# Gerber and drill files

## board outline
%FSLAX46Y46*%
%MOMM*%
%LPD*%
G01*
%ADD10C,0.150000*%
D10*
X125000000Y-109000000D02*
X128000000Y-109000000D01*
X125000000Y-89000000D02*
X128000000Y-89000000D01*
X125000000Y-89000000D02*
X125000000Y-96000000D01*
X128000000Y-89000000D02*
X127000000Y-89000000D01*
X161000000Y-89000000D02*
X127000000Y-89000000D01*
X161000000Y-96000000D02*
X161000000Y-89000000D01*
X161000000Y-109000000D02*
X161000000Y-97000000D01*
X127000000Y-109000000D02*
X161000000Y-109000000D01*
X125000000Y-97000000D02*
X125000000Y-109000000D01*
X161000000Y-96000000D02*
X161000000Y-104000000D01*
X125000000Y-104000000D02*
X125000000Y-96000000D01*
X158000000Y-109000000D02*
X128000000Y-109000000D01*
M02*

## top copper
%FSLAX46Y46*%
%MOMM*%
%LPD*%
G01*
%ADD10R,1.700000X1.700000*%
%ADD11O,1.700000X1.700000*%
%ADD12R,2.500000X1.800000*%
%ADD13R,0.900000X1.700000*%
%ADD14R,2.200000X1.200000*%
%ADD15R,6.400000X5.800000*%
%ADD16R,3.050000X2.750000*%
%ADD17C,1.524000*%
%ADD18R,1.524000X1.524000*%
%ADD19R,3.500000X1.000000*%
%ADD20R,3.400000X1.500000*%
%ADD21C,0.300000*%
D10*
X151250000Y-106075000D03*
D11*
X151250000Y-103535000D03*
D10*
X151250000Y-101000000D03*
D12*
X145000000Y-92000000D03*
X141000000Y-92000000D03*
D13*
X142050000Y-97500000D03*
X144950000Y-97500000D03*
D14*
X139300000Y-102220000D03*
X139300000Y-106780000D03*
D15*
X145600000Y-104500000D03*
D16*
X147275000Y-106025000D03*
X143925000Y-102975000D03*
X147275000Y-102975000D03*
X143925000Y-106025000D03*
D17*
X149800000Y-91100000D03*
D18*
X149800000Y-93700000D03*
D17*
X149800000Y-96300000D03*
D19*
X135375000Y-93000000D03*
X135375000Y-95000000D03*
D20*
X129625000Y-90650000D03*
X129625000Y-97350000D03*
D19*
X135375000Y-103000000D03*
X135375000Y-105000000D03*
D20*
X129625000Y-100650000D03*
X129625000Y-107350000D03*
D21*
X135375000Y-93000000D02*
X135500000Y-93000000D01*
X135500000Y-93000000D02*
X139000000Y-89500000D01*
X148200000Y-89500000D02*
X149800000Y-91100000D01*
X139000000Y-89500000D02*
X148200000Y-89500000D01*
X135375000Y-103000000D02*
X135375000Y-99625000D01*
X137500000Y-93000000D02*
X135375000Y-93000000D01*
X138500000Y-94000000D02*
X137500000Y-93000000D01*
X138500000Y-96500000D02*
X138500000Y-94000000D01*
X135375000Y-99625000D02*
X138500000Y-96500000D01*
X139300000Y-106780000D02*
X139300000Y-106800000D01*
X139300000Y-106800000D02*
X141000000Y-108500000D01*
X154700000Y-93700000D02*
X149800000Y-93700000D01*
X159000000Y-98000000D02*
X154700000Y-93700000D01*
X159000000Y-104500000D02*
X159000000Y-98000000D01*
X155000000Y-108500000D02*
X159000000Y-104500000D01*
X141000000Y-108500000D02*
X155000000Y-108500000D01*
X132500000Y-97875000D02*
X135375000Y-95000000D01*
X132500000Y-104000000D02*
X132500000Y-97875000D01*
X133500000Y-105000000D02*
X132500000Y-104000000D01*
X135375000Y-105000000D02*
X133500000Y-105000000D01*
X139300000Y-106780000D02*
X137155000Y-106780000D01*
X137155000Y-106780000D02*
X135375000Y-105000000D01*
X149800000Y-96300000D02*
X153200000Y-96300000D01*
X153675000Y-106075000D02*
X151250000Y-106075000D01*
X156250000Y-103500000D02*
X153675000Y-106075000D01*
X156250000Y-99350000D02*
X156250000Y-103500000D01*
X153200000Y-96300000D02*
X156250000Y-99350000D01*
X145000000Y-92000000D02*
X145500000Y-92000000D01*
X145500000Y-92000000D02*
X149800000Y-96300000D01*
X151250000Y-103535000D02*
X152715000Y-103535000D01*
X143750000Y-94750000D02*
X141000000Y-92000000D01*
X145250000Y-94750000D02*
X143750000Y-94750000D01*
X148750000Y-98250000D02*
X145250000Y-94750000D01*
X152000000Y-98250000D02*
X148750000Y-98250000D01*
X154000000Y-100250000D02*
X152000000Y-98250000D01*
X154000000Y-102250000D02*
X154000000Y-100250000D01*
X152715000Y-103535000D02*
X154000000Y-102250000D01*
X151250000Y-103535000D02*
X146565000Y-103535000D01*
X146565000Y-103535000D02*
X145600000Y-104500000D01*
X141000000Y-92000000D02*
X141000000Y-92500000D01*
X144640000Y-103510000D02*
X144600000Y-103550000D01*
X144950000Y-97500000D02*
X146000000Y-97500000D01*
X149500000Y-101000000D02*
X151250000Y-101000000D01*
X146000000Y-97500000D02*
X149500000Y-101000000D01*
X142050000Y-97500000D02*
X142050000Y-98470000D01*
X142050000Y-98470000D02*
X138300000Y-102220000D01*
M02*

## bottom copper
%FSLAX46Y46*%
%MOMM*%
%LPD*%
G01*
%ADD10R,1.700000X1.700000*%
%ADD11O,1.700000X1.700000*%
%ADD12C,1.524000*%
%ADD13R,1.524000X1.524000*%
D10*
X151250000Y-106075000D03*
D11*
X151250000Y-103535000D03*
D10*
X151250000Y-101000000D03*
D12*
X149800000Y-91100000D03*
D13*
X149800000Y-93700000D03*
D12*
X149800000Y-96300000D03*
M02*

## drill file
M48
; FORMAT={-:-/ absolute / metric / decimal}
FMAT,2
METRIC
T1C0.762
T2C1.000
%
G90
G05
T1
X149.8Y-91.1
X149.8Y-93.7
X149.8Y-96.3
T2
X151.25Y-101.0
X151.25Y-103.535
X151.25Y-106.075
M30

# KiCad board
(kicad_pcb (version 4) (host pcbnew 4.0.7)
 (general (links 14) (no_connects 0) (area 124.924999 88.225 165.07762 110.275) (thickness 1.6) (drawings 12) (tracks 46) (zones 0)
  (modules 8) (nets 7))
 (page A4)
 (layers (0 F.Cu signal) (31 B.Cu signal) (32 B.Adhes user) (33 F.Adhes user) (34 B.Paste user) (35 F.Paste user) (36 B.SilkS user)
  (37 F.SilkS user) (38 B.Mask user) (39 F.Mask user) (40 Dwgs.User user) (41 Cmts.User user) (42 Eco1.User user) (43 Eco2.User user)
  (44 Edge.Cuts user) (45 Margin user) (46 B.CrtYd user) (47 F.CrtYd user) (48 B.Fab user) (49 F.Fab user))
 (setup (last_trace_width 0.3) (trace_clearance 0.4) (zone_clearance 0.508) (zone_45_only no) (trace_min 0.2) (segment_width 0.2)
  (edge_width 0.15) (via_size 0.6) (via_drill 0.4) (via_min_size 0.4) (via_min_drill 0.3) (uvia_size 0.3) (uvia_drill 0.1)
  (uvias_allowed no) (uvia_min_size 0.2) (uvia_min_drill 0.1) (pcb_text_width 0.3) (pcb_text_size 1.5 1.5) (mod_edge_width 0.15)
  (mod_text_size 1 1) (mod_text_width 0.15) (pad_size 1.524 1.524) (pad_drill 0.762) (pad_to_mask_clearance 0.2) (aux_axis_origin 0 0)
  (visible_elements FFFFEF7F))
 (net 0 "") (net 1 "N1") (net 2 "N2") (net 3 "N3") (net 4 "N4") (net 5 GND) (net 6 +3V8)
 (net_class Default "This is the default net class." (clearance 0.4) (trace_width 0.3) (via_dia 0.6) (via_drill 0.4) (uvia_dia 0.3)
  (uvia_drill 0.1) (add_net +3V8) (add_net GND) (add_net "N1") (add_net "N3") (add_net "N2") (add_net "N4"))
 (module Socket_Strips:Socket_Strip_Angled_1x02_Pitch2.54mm (layer F.Cu) (at 151.25 106.075 180)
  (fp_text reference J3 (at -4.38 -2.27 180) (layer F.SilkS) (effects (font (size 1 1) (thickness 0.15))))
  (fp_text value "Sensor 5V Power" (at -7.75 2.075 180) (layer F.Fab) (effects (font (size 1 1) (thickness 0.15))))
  (pad 1 thru_hole rect (at 0 0 180) (size 1.7 1.7) (drill 1) (layers *.Cu *.Mask) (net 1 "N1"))
  (pad 2 thru_hole oval (at 0 2.54 180) (size 1.7 1.7) (drill 1) (layers *.Cu *.Mask)))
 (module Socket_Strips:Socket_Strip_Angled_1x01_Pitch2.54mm (layer F.Cu) (at 151.25 101 180)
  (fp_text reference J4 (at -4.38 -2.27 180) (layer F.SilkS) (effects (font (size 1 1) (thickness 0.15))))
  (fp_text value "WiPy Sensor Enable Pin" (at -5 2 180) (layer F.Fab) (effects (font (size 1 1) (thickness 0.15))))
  (pad 1 thru_hole rect (at 0 0 180) (size 1.7 1.7) (drill 1) (layers *.Cu *.Mask) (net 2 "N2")))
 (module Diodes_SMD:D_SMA (layer F.Cu) (at 143 92 180)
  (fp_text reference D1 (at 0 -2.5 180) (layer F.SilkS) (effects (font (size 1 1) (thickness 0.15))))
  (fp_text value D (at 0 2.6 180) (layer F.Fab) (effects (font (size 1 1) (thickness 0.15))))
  (pad 1 smd rect (at -2 0 180) (size 2.5 1.8) (layers F.Cu F.Paste F.Mask) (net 1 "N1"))
  (pad 2 smd rect (at 2 0 180) (size 2.5 1.8) (layers F.Cu F.Paste F.Mask) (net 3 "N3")))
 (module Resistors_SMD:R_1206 (layer F.Cu) (at 143.5 97.5)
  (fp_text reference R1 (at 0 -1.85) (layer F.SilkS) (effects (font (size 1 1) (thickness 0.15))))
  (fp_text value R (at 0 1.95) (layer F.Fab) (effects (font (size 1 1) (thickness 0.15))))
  (pad 1 smd rect (at -1.45 0) (size 0.9 1.7) (layers F.Cu F.Paste F.Mask) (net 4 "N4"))
  (pad 2 smd rect (at 1.45 0) (size 0.9 1.7) (layers F.Cu F.Paste F.Mask) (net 2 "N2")))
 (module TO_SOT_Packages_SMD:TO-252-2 (layer F.Cu) (at 143.5 104.5)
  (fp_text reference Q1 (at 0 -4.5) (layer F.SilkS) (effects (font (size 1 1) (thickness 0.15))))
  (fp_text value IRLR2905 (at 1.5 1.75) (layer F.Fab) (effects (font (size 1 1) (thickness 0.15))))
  (pad 1 smd rect (at -4.2 -2.28) (size 2.2 1.2) (layers F.Cu F.Paste F.Mask) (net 4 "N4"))
  (pad 3 smd rect (at -4.2 2.28) (size 2.2 1.2) (layers F.Cu F.Paste F.Mask) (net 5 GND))
  (pad 2 smd rect (at 2.1 0) (size 6.4 5.8) (layers F.Cu F.Mask) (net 3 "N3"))
  (pad 2 smd rect (at 3.775 1.525) (size 3.05 2.75) (layers F.Cu F.Paste) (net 3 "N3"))
  (pad 2 smd rect (at 0.425 -1.525) (size 3.05 2.75) (layers F.Cu F.Paste) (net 3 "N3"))
  (pad 2 smd rect (at 3.775 -1.525) (size 3.05 2.75) (layers F.Cu F.Paste) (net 3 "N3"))
  (pad 2 smd rect (at 0.425 1.525) (size 3.05 2.75) (layers F.Cu F.Paste) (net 3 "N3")))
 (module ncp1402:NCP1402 (layer F.Cu) (at 161 89.5 180)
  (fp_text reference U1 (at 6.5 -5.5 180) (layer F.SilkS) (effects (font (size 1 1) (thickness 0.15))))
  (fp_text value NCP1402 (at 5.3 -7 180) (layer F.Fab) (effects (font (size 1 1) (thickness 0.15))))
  (pad 1 thru_hole circle (at 11.2 -1.6 180) (size 1.524 1.524) (drill 0.762) (layers *.Cu *.Mask) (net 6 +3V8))
  (pad 2 thru_hole rect (at 11.2 -4.2 180) (size 1.524 1.524) (drill 0.762) (layers *.Cu *.Mask) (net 5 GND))
  (pad 3 thru_hole circle (at 11.2 -6.8 180) (size 1.524 1.524) (drill 0.762) (layers *.Cu *.Mask) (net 1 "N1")))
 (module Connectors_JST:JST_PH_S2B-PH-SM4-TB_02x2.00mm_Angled (layer F.Cu) (at 132.5 94 270)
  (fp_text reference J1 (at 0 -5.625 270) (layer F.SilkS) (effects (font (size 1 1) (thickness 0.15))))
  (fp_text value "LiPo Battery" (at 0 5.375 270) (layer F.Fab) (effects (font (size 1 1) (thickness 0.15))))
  (pad 1 smd rect (at -1 -2.875 270) (size 1 3.5) (layers F.Cu F.Paste F.Mask) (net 6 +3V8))
  (pad 2 smd rect (at 1 -2.875 270) (size 1 3.5) (layers F.Cu F.Paste F.Mask) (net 5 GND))
  (pad "" smd rect (at -3.35 2.875 270) (size 1.5 3.4) (layers F.Cu F.Paste F.Mask))
  (pad "" smd rect (at 3.35 2.875 270) (size 1.5 3.4) (layers F.Cu F.Paste F.Mask)))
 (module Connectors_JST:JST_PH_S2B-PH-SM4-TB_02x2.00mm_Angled (layer F.Cu) (at 132.5 104 270)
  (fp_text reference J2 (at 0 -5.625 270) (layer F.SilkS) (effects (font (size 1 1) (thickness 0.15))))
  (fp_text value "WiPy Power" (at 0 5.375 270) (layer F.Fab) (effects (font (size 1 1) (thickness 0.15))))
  (pad 1 smd rect (at -1 -2.875 270) (size 1 3.5) (layers F.Cu F.Paste F.Mask) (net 6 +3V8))
  (pad 2 smd rect (at 1 -2.875 270) (size 1 3.5) (layers F.Cu F.Paste F.Mask) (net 5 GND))
  (pad "" smd rect (at -3.35 2.875 270) (size 1.5 3.4) (layers F.Cu F.Paste F.Mask))
  (pad "" smd rect (at 3.35 2.875 270) (size 1.5 3.4) (layers F.Cu F.Paste F.Mask)))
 (gr_line (start 125 109) (end 128 109) (angle 90) (layer Edge.Cuts) (width 0.15))
 (gr_line (start 125 89) (end 128 89) (angle 90) (layer Edge.Cuts) (width 0.15))
 (gr_line (start 125 89) (end 125 96) (angle 90) (layer Edge.Cuts) (width 0.15))
 (gr_line (start 128 89) (end 127 89) (angle 90) (layer Edge.Cuts) (width 0.15))
 (gr_line (start 161 89) (end 127 89) (angle 90) (layer Edge.Cuts) (width 0.15))
 (gr_line (start 161 96) (end 161 89) (angle 90) (layer Edge.Cuts) (width 0.15))
 (gr_line (start 161 109) (end 161 97) (angle 90) (layer Edge.Cuts) (width 0.15))
 (gr_line (start 127 109) (end 161 109) (angle 90) (layer Edge.Cuts) (width 0.15))
 (gr_line (start 125 97) (end 125 109) (angle 90) (layer Edge.Cuts) (width 0.15))
 (gr_line (start 161 96) (end 161 104) (angle 90) (layer Edge.Cuts) (width 0.15))
 (gr_line (start 125 104) (end 125 96) (angle 90) (layer Edge.Cuts) (width 0.15))
 (gr_line (start 158 109) (end 128 109) (angle 90) (layer Edge.Cuts) (width 0.15))
 (segment (start 135.375 93) (end 135.5 93) (width 0.3) (layer F.Cu) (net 6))
 (segment (start 135.5 93) (end 139 89.5) (width 0.3) (layer F.Cu) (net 6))
 (segment (start 148.2 89.5) (end 149.8 91.1) (width 0.3) (layer F.Cu) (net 6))
 (segment (start 139 89.5) (end 148.2 89.5) (width 0.3) (layer F.Cu) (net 6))
 (segment (start 135.375 103) (end 135.375 99.625) (width 0.3) (layer F.Cu) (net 6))
 (segment (start 137.5 93) (end 135.375 93) (width 0.3) (layer F.Cu) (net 6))
 (segment (start 138.5 94) (end 137.5 93) (width 0.3) (layer F.Cu) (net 6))
 (segment (start 138.5 96.5) (end 138.5 94) (width 0.3) (layer F.Cu) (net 6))
 (segment (start 135.375 99.625) (end 138.5 96.5) (width 0.3) (layer F.Cu) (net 6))
 (segment (start 139.3 106.78) (end 139.3 106.8) (width 0.3) (layer F.Cu) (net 5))
 (segment (start 139.3 106.8) (end 141 108.5) (width 0.3) (layer F.Cu) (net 5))
 (segment (start 154.7 93.7) (end 149.8 93.7) (width 0.3) (layer F.Cu) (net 5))
 (segment (start 159 98) (end 154.7 93.7) (width 0.3) (layer F.Cu) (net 5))
 (segment (start 159 104.5) (end 159 98) (width 0.3) (layer F.Cu) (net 5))
 (segment (start 155 108.5) (end 159 104.5) (width 0.3) (layer F.Cu) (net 5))
 (segment (start 141 108.5) (end 155 108.5) (width 0.3) (layer F.Cu) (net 5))
 (segment (start 132.5 97.875) (end 135.375 95) (width 0.3) (layer F.Cu) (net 5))
 (segment (start 132.5 104) (end 132.5 97.875) (width 0.3) (layer F.Cu) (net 5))
 (segment (start 133.5 105) (end 132.5 104) (width 0.3) (layer F.Cu) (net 5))
 (segment (start 135.375 105) (end 133.5 105) (width 0.3) (layer F.Cu) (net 5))
 (segment (start 139.3 106.78) (end 137.155 106.78) (width 0.3) (layer F.Cu) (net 5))
 (segment (start 137.155 106.78) (end 135.375 105) (width 0.3) (layer F.Cu) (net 5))
 (segment (start 149.8 96.3) (end 153.2 96.3) (width 0.3) (layer F.Cu) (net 1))
 (segment (start 153.675 106.075) (end 151.25 106.075) (width 0.3) (layer F.Cu) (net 1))
 (segment (start 156.25 103.5) (end 153.675 106.075) (width 0.3) (layer F.Cu) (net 1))
 (segment (start 156.25 99.35) (end 156.25 103.5) (width 0.3) (layer F.Cu) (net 1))
 (segment (start 153.2 96.3) (end 156.25 99.35) (width 0.3) (layer F.Cu) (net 1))
 (segment (start 145 92) (end 145.5 92) (width 0.3) (layer F.Cu) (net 1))
 (segment (start 145.5 92) (end 149.8 96.3) (width 0.3) (layer F.Cu) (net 1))
 (segment (start 151.25 103.535) (end 152.715 103.535) (width 0.3) (layer F.Cu) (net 3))
 (segment (start 143.75 94.75) (end 141 92) (width 0.3) (layer F.Cu) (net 3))
 (segment (start 145.25 94.75) (end 143.75 94.75) (width 0.3) (layer F.Cu) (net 3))
 (segment (start 148.75 98.25) (end 145.25 94.75) (width 0.3) (layer F.Cu) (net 3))
 (segment (start 152 98.25) (end 148.75 98.25) (width 0.3) (layer F.Cu) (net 3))
 (segment (start 154 100.25) (end 152 98.25) (width 0.3) (layer F.Cu) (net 3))
 (segment (start 154 102.25) (end 154 100.25) (width 0.3) (layer F.Cu) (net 3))
 (segment (start 152.715 103.535) (end 154 102.25) (width 0.3) (layer F.Cu) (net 3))
 (segment (start 151.25 103.535) (end 146.565 103.535) (width 0.3) (layer F.Cu) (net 3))
 (segment (start 146.565 103.535) (end 145.6 104.5) (width 0.3) (layer F.Cu) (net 3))
 (segment (start 141 92) (end 141 92.5) (width 0.3) (layer F.Cu) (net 3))
 (segment (start 144.64 103.51) (end 144.6 103.55) (width 0.3) (layer F.Cu) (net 3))
 (segment (start 144.95 97.5) (end 146 97.5) (width 0.3) (layer F.Cu) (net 2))
 (segment (start 149.5 101) (end 151.25 101) (width 0.3) (layer F.Cu) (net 2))
 (segment (start 146 97.5) (end 149.5 101) (width 0.3) (layer F.Cu) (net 2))
 (segment (start 142.05 97.5) (end 142.05 98.47) (width 0.3) (layer F.Cu) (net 4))
 (segment (start 142.05 98.47) (end 138.3 102.22) (width 0.3) (layer F.Cu) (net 4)))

